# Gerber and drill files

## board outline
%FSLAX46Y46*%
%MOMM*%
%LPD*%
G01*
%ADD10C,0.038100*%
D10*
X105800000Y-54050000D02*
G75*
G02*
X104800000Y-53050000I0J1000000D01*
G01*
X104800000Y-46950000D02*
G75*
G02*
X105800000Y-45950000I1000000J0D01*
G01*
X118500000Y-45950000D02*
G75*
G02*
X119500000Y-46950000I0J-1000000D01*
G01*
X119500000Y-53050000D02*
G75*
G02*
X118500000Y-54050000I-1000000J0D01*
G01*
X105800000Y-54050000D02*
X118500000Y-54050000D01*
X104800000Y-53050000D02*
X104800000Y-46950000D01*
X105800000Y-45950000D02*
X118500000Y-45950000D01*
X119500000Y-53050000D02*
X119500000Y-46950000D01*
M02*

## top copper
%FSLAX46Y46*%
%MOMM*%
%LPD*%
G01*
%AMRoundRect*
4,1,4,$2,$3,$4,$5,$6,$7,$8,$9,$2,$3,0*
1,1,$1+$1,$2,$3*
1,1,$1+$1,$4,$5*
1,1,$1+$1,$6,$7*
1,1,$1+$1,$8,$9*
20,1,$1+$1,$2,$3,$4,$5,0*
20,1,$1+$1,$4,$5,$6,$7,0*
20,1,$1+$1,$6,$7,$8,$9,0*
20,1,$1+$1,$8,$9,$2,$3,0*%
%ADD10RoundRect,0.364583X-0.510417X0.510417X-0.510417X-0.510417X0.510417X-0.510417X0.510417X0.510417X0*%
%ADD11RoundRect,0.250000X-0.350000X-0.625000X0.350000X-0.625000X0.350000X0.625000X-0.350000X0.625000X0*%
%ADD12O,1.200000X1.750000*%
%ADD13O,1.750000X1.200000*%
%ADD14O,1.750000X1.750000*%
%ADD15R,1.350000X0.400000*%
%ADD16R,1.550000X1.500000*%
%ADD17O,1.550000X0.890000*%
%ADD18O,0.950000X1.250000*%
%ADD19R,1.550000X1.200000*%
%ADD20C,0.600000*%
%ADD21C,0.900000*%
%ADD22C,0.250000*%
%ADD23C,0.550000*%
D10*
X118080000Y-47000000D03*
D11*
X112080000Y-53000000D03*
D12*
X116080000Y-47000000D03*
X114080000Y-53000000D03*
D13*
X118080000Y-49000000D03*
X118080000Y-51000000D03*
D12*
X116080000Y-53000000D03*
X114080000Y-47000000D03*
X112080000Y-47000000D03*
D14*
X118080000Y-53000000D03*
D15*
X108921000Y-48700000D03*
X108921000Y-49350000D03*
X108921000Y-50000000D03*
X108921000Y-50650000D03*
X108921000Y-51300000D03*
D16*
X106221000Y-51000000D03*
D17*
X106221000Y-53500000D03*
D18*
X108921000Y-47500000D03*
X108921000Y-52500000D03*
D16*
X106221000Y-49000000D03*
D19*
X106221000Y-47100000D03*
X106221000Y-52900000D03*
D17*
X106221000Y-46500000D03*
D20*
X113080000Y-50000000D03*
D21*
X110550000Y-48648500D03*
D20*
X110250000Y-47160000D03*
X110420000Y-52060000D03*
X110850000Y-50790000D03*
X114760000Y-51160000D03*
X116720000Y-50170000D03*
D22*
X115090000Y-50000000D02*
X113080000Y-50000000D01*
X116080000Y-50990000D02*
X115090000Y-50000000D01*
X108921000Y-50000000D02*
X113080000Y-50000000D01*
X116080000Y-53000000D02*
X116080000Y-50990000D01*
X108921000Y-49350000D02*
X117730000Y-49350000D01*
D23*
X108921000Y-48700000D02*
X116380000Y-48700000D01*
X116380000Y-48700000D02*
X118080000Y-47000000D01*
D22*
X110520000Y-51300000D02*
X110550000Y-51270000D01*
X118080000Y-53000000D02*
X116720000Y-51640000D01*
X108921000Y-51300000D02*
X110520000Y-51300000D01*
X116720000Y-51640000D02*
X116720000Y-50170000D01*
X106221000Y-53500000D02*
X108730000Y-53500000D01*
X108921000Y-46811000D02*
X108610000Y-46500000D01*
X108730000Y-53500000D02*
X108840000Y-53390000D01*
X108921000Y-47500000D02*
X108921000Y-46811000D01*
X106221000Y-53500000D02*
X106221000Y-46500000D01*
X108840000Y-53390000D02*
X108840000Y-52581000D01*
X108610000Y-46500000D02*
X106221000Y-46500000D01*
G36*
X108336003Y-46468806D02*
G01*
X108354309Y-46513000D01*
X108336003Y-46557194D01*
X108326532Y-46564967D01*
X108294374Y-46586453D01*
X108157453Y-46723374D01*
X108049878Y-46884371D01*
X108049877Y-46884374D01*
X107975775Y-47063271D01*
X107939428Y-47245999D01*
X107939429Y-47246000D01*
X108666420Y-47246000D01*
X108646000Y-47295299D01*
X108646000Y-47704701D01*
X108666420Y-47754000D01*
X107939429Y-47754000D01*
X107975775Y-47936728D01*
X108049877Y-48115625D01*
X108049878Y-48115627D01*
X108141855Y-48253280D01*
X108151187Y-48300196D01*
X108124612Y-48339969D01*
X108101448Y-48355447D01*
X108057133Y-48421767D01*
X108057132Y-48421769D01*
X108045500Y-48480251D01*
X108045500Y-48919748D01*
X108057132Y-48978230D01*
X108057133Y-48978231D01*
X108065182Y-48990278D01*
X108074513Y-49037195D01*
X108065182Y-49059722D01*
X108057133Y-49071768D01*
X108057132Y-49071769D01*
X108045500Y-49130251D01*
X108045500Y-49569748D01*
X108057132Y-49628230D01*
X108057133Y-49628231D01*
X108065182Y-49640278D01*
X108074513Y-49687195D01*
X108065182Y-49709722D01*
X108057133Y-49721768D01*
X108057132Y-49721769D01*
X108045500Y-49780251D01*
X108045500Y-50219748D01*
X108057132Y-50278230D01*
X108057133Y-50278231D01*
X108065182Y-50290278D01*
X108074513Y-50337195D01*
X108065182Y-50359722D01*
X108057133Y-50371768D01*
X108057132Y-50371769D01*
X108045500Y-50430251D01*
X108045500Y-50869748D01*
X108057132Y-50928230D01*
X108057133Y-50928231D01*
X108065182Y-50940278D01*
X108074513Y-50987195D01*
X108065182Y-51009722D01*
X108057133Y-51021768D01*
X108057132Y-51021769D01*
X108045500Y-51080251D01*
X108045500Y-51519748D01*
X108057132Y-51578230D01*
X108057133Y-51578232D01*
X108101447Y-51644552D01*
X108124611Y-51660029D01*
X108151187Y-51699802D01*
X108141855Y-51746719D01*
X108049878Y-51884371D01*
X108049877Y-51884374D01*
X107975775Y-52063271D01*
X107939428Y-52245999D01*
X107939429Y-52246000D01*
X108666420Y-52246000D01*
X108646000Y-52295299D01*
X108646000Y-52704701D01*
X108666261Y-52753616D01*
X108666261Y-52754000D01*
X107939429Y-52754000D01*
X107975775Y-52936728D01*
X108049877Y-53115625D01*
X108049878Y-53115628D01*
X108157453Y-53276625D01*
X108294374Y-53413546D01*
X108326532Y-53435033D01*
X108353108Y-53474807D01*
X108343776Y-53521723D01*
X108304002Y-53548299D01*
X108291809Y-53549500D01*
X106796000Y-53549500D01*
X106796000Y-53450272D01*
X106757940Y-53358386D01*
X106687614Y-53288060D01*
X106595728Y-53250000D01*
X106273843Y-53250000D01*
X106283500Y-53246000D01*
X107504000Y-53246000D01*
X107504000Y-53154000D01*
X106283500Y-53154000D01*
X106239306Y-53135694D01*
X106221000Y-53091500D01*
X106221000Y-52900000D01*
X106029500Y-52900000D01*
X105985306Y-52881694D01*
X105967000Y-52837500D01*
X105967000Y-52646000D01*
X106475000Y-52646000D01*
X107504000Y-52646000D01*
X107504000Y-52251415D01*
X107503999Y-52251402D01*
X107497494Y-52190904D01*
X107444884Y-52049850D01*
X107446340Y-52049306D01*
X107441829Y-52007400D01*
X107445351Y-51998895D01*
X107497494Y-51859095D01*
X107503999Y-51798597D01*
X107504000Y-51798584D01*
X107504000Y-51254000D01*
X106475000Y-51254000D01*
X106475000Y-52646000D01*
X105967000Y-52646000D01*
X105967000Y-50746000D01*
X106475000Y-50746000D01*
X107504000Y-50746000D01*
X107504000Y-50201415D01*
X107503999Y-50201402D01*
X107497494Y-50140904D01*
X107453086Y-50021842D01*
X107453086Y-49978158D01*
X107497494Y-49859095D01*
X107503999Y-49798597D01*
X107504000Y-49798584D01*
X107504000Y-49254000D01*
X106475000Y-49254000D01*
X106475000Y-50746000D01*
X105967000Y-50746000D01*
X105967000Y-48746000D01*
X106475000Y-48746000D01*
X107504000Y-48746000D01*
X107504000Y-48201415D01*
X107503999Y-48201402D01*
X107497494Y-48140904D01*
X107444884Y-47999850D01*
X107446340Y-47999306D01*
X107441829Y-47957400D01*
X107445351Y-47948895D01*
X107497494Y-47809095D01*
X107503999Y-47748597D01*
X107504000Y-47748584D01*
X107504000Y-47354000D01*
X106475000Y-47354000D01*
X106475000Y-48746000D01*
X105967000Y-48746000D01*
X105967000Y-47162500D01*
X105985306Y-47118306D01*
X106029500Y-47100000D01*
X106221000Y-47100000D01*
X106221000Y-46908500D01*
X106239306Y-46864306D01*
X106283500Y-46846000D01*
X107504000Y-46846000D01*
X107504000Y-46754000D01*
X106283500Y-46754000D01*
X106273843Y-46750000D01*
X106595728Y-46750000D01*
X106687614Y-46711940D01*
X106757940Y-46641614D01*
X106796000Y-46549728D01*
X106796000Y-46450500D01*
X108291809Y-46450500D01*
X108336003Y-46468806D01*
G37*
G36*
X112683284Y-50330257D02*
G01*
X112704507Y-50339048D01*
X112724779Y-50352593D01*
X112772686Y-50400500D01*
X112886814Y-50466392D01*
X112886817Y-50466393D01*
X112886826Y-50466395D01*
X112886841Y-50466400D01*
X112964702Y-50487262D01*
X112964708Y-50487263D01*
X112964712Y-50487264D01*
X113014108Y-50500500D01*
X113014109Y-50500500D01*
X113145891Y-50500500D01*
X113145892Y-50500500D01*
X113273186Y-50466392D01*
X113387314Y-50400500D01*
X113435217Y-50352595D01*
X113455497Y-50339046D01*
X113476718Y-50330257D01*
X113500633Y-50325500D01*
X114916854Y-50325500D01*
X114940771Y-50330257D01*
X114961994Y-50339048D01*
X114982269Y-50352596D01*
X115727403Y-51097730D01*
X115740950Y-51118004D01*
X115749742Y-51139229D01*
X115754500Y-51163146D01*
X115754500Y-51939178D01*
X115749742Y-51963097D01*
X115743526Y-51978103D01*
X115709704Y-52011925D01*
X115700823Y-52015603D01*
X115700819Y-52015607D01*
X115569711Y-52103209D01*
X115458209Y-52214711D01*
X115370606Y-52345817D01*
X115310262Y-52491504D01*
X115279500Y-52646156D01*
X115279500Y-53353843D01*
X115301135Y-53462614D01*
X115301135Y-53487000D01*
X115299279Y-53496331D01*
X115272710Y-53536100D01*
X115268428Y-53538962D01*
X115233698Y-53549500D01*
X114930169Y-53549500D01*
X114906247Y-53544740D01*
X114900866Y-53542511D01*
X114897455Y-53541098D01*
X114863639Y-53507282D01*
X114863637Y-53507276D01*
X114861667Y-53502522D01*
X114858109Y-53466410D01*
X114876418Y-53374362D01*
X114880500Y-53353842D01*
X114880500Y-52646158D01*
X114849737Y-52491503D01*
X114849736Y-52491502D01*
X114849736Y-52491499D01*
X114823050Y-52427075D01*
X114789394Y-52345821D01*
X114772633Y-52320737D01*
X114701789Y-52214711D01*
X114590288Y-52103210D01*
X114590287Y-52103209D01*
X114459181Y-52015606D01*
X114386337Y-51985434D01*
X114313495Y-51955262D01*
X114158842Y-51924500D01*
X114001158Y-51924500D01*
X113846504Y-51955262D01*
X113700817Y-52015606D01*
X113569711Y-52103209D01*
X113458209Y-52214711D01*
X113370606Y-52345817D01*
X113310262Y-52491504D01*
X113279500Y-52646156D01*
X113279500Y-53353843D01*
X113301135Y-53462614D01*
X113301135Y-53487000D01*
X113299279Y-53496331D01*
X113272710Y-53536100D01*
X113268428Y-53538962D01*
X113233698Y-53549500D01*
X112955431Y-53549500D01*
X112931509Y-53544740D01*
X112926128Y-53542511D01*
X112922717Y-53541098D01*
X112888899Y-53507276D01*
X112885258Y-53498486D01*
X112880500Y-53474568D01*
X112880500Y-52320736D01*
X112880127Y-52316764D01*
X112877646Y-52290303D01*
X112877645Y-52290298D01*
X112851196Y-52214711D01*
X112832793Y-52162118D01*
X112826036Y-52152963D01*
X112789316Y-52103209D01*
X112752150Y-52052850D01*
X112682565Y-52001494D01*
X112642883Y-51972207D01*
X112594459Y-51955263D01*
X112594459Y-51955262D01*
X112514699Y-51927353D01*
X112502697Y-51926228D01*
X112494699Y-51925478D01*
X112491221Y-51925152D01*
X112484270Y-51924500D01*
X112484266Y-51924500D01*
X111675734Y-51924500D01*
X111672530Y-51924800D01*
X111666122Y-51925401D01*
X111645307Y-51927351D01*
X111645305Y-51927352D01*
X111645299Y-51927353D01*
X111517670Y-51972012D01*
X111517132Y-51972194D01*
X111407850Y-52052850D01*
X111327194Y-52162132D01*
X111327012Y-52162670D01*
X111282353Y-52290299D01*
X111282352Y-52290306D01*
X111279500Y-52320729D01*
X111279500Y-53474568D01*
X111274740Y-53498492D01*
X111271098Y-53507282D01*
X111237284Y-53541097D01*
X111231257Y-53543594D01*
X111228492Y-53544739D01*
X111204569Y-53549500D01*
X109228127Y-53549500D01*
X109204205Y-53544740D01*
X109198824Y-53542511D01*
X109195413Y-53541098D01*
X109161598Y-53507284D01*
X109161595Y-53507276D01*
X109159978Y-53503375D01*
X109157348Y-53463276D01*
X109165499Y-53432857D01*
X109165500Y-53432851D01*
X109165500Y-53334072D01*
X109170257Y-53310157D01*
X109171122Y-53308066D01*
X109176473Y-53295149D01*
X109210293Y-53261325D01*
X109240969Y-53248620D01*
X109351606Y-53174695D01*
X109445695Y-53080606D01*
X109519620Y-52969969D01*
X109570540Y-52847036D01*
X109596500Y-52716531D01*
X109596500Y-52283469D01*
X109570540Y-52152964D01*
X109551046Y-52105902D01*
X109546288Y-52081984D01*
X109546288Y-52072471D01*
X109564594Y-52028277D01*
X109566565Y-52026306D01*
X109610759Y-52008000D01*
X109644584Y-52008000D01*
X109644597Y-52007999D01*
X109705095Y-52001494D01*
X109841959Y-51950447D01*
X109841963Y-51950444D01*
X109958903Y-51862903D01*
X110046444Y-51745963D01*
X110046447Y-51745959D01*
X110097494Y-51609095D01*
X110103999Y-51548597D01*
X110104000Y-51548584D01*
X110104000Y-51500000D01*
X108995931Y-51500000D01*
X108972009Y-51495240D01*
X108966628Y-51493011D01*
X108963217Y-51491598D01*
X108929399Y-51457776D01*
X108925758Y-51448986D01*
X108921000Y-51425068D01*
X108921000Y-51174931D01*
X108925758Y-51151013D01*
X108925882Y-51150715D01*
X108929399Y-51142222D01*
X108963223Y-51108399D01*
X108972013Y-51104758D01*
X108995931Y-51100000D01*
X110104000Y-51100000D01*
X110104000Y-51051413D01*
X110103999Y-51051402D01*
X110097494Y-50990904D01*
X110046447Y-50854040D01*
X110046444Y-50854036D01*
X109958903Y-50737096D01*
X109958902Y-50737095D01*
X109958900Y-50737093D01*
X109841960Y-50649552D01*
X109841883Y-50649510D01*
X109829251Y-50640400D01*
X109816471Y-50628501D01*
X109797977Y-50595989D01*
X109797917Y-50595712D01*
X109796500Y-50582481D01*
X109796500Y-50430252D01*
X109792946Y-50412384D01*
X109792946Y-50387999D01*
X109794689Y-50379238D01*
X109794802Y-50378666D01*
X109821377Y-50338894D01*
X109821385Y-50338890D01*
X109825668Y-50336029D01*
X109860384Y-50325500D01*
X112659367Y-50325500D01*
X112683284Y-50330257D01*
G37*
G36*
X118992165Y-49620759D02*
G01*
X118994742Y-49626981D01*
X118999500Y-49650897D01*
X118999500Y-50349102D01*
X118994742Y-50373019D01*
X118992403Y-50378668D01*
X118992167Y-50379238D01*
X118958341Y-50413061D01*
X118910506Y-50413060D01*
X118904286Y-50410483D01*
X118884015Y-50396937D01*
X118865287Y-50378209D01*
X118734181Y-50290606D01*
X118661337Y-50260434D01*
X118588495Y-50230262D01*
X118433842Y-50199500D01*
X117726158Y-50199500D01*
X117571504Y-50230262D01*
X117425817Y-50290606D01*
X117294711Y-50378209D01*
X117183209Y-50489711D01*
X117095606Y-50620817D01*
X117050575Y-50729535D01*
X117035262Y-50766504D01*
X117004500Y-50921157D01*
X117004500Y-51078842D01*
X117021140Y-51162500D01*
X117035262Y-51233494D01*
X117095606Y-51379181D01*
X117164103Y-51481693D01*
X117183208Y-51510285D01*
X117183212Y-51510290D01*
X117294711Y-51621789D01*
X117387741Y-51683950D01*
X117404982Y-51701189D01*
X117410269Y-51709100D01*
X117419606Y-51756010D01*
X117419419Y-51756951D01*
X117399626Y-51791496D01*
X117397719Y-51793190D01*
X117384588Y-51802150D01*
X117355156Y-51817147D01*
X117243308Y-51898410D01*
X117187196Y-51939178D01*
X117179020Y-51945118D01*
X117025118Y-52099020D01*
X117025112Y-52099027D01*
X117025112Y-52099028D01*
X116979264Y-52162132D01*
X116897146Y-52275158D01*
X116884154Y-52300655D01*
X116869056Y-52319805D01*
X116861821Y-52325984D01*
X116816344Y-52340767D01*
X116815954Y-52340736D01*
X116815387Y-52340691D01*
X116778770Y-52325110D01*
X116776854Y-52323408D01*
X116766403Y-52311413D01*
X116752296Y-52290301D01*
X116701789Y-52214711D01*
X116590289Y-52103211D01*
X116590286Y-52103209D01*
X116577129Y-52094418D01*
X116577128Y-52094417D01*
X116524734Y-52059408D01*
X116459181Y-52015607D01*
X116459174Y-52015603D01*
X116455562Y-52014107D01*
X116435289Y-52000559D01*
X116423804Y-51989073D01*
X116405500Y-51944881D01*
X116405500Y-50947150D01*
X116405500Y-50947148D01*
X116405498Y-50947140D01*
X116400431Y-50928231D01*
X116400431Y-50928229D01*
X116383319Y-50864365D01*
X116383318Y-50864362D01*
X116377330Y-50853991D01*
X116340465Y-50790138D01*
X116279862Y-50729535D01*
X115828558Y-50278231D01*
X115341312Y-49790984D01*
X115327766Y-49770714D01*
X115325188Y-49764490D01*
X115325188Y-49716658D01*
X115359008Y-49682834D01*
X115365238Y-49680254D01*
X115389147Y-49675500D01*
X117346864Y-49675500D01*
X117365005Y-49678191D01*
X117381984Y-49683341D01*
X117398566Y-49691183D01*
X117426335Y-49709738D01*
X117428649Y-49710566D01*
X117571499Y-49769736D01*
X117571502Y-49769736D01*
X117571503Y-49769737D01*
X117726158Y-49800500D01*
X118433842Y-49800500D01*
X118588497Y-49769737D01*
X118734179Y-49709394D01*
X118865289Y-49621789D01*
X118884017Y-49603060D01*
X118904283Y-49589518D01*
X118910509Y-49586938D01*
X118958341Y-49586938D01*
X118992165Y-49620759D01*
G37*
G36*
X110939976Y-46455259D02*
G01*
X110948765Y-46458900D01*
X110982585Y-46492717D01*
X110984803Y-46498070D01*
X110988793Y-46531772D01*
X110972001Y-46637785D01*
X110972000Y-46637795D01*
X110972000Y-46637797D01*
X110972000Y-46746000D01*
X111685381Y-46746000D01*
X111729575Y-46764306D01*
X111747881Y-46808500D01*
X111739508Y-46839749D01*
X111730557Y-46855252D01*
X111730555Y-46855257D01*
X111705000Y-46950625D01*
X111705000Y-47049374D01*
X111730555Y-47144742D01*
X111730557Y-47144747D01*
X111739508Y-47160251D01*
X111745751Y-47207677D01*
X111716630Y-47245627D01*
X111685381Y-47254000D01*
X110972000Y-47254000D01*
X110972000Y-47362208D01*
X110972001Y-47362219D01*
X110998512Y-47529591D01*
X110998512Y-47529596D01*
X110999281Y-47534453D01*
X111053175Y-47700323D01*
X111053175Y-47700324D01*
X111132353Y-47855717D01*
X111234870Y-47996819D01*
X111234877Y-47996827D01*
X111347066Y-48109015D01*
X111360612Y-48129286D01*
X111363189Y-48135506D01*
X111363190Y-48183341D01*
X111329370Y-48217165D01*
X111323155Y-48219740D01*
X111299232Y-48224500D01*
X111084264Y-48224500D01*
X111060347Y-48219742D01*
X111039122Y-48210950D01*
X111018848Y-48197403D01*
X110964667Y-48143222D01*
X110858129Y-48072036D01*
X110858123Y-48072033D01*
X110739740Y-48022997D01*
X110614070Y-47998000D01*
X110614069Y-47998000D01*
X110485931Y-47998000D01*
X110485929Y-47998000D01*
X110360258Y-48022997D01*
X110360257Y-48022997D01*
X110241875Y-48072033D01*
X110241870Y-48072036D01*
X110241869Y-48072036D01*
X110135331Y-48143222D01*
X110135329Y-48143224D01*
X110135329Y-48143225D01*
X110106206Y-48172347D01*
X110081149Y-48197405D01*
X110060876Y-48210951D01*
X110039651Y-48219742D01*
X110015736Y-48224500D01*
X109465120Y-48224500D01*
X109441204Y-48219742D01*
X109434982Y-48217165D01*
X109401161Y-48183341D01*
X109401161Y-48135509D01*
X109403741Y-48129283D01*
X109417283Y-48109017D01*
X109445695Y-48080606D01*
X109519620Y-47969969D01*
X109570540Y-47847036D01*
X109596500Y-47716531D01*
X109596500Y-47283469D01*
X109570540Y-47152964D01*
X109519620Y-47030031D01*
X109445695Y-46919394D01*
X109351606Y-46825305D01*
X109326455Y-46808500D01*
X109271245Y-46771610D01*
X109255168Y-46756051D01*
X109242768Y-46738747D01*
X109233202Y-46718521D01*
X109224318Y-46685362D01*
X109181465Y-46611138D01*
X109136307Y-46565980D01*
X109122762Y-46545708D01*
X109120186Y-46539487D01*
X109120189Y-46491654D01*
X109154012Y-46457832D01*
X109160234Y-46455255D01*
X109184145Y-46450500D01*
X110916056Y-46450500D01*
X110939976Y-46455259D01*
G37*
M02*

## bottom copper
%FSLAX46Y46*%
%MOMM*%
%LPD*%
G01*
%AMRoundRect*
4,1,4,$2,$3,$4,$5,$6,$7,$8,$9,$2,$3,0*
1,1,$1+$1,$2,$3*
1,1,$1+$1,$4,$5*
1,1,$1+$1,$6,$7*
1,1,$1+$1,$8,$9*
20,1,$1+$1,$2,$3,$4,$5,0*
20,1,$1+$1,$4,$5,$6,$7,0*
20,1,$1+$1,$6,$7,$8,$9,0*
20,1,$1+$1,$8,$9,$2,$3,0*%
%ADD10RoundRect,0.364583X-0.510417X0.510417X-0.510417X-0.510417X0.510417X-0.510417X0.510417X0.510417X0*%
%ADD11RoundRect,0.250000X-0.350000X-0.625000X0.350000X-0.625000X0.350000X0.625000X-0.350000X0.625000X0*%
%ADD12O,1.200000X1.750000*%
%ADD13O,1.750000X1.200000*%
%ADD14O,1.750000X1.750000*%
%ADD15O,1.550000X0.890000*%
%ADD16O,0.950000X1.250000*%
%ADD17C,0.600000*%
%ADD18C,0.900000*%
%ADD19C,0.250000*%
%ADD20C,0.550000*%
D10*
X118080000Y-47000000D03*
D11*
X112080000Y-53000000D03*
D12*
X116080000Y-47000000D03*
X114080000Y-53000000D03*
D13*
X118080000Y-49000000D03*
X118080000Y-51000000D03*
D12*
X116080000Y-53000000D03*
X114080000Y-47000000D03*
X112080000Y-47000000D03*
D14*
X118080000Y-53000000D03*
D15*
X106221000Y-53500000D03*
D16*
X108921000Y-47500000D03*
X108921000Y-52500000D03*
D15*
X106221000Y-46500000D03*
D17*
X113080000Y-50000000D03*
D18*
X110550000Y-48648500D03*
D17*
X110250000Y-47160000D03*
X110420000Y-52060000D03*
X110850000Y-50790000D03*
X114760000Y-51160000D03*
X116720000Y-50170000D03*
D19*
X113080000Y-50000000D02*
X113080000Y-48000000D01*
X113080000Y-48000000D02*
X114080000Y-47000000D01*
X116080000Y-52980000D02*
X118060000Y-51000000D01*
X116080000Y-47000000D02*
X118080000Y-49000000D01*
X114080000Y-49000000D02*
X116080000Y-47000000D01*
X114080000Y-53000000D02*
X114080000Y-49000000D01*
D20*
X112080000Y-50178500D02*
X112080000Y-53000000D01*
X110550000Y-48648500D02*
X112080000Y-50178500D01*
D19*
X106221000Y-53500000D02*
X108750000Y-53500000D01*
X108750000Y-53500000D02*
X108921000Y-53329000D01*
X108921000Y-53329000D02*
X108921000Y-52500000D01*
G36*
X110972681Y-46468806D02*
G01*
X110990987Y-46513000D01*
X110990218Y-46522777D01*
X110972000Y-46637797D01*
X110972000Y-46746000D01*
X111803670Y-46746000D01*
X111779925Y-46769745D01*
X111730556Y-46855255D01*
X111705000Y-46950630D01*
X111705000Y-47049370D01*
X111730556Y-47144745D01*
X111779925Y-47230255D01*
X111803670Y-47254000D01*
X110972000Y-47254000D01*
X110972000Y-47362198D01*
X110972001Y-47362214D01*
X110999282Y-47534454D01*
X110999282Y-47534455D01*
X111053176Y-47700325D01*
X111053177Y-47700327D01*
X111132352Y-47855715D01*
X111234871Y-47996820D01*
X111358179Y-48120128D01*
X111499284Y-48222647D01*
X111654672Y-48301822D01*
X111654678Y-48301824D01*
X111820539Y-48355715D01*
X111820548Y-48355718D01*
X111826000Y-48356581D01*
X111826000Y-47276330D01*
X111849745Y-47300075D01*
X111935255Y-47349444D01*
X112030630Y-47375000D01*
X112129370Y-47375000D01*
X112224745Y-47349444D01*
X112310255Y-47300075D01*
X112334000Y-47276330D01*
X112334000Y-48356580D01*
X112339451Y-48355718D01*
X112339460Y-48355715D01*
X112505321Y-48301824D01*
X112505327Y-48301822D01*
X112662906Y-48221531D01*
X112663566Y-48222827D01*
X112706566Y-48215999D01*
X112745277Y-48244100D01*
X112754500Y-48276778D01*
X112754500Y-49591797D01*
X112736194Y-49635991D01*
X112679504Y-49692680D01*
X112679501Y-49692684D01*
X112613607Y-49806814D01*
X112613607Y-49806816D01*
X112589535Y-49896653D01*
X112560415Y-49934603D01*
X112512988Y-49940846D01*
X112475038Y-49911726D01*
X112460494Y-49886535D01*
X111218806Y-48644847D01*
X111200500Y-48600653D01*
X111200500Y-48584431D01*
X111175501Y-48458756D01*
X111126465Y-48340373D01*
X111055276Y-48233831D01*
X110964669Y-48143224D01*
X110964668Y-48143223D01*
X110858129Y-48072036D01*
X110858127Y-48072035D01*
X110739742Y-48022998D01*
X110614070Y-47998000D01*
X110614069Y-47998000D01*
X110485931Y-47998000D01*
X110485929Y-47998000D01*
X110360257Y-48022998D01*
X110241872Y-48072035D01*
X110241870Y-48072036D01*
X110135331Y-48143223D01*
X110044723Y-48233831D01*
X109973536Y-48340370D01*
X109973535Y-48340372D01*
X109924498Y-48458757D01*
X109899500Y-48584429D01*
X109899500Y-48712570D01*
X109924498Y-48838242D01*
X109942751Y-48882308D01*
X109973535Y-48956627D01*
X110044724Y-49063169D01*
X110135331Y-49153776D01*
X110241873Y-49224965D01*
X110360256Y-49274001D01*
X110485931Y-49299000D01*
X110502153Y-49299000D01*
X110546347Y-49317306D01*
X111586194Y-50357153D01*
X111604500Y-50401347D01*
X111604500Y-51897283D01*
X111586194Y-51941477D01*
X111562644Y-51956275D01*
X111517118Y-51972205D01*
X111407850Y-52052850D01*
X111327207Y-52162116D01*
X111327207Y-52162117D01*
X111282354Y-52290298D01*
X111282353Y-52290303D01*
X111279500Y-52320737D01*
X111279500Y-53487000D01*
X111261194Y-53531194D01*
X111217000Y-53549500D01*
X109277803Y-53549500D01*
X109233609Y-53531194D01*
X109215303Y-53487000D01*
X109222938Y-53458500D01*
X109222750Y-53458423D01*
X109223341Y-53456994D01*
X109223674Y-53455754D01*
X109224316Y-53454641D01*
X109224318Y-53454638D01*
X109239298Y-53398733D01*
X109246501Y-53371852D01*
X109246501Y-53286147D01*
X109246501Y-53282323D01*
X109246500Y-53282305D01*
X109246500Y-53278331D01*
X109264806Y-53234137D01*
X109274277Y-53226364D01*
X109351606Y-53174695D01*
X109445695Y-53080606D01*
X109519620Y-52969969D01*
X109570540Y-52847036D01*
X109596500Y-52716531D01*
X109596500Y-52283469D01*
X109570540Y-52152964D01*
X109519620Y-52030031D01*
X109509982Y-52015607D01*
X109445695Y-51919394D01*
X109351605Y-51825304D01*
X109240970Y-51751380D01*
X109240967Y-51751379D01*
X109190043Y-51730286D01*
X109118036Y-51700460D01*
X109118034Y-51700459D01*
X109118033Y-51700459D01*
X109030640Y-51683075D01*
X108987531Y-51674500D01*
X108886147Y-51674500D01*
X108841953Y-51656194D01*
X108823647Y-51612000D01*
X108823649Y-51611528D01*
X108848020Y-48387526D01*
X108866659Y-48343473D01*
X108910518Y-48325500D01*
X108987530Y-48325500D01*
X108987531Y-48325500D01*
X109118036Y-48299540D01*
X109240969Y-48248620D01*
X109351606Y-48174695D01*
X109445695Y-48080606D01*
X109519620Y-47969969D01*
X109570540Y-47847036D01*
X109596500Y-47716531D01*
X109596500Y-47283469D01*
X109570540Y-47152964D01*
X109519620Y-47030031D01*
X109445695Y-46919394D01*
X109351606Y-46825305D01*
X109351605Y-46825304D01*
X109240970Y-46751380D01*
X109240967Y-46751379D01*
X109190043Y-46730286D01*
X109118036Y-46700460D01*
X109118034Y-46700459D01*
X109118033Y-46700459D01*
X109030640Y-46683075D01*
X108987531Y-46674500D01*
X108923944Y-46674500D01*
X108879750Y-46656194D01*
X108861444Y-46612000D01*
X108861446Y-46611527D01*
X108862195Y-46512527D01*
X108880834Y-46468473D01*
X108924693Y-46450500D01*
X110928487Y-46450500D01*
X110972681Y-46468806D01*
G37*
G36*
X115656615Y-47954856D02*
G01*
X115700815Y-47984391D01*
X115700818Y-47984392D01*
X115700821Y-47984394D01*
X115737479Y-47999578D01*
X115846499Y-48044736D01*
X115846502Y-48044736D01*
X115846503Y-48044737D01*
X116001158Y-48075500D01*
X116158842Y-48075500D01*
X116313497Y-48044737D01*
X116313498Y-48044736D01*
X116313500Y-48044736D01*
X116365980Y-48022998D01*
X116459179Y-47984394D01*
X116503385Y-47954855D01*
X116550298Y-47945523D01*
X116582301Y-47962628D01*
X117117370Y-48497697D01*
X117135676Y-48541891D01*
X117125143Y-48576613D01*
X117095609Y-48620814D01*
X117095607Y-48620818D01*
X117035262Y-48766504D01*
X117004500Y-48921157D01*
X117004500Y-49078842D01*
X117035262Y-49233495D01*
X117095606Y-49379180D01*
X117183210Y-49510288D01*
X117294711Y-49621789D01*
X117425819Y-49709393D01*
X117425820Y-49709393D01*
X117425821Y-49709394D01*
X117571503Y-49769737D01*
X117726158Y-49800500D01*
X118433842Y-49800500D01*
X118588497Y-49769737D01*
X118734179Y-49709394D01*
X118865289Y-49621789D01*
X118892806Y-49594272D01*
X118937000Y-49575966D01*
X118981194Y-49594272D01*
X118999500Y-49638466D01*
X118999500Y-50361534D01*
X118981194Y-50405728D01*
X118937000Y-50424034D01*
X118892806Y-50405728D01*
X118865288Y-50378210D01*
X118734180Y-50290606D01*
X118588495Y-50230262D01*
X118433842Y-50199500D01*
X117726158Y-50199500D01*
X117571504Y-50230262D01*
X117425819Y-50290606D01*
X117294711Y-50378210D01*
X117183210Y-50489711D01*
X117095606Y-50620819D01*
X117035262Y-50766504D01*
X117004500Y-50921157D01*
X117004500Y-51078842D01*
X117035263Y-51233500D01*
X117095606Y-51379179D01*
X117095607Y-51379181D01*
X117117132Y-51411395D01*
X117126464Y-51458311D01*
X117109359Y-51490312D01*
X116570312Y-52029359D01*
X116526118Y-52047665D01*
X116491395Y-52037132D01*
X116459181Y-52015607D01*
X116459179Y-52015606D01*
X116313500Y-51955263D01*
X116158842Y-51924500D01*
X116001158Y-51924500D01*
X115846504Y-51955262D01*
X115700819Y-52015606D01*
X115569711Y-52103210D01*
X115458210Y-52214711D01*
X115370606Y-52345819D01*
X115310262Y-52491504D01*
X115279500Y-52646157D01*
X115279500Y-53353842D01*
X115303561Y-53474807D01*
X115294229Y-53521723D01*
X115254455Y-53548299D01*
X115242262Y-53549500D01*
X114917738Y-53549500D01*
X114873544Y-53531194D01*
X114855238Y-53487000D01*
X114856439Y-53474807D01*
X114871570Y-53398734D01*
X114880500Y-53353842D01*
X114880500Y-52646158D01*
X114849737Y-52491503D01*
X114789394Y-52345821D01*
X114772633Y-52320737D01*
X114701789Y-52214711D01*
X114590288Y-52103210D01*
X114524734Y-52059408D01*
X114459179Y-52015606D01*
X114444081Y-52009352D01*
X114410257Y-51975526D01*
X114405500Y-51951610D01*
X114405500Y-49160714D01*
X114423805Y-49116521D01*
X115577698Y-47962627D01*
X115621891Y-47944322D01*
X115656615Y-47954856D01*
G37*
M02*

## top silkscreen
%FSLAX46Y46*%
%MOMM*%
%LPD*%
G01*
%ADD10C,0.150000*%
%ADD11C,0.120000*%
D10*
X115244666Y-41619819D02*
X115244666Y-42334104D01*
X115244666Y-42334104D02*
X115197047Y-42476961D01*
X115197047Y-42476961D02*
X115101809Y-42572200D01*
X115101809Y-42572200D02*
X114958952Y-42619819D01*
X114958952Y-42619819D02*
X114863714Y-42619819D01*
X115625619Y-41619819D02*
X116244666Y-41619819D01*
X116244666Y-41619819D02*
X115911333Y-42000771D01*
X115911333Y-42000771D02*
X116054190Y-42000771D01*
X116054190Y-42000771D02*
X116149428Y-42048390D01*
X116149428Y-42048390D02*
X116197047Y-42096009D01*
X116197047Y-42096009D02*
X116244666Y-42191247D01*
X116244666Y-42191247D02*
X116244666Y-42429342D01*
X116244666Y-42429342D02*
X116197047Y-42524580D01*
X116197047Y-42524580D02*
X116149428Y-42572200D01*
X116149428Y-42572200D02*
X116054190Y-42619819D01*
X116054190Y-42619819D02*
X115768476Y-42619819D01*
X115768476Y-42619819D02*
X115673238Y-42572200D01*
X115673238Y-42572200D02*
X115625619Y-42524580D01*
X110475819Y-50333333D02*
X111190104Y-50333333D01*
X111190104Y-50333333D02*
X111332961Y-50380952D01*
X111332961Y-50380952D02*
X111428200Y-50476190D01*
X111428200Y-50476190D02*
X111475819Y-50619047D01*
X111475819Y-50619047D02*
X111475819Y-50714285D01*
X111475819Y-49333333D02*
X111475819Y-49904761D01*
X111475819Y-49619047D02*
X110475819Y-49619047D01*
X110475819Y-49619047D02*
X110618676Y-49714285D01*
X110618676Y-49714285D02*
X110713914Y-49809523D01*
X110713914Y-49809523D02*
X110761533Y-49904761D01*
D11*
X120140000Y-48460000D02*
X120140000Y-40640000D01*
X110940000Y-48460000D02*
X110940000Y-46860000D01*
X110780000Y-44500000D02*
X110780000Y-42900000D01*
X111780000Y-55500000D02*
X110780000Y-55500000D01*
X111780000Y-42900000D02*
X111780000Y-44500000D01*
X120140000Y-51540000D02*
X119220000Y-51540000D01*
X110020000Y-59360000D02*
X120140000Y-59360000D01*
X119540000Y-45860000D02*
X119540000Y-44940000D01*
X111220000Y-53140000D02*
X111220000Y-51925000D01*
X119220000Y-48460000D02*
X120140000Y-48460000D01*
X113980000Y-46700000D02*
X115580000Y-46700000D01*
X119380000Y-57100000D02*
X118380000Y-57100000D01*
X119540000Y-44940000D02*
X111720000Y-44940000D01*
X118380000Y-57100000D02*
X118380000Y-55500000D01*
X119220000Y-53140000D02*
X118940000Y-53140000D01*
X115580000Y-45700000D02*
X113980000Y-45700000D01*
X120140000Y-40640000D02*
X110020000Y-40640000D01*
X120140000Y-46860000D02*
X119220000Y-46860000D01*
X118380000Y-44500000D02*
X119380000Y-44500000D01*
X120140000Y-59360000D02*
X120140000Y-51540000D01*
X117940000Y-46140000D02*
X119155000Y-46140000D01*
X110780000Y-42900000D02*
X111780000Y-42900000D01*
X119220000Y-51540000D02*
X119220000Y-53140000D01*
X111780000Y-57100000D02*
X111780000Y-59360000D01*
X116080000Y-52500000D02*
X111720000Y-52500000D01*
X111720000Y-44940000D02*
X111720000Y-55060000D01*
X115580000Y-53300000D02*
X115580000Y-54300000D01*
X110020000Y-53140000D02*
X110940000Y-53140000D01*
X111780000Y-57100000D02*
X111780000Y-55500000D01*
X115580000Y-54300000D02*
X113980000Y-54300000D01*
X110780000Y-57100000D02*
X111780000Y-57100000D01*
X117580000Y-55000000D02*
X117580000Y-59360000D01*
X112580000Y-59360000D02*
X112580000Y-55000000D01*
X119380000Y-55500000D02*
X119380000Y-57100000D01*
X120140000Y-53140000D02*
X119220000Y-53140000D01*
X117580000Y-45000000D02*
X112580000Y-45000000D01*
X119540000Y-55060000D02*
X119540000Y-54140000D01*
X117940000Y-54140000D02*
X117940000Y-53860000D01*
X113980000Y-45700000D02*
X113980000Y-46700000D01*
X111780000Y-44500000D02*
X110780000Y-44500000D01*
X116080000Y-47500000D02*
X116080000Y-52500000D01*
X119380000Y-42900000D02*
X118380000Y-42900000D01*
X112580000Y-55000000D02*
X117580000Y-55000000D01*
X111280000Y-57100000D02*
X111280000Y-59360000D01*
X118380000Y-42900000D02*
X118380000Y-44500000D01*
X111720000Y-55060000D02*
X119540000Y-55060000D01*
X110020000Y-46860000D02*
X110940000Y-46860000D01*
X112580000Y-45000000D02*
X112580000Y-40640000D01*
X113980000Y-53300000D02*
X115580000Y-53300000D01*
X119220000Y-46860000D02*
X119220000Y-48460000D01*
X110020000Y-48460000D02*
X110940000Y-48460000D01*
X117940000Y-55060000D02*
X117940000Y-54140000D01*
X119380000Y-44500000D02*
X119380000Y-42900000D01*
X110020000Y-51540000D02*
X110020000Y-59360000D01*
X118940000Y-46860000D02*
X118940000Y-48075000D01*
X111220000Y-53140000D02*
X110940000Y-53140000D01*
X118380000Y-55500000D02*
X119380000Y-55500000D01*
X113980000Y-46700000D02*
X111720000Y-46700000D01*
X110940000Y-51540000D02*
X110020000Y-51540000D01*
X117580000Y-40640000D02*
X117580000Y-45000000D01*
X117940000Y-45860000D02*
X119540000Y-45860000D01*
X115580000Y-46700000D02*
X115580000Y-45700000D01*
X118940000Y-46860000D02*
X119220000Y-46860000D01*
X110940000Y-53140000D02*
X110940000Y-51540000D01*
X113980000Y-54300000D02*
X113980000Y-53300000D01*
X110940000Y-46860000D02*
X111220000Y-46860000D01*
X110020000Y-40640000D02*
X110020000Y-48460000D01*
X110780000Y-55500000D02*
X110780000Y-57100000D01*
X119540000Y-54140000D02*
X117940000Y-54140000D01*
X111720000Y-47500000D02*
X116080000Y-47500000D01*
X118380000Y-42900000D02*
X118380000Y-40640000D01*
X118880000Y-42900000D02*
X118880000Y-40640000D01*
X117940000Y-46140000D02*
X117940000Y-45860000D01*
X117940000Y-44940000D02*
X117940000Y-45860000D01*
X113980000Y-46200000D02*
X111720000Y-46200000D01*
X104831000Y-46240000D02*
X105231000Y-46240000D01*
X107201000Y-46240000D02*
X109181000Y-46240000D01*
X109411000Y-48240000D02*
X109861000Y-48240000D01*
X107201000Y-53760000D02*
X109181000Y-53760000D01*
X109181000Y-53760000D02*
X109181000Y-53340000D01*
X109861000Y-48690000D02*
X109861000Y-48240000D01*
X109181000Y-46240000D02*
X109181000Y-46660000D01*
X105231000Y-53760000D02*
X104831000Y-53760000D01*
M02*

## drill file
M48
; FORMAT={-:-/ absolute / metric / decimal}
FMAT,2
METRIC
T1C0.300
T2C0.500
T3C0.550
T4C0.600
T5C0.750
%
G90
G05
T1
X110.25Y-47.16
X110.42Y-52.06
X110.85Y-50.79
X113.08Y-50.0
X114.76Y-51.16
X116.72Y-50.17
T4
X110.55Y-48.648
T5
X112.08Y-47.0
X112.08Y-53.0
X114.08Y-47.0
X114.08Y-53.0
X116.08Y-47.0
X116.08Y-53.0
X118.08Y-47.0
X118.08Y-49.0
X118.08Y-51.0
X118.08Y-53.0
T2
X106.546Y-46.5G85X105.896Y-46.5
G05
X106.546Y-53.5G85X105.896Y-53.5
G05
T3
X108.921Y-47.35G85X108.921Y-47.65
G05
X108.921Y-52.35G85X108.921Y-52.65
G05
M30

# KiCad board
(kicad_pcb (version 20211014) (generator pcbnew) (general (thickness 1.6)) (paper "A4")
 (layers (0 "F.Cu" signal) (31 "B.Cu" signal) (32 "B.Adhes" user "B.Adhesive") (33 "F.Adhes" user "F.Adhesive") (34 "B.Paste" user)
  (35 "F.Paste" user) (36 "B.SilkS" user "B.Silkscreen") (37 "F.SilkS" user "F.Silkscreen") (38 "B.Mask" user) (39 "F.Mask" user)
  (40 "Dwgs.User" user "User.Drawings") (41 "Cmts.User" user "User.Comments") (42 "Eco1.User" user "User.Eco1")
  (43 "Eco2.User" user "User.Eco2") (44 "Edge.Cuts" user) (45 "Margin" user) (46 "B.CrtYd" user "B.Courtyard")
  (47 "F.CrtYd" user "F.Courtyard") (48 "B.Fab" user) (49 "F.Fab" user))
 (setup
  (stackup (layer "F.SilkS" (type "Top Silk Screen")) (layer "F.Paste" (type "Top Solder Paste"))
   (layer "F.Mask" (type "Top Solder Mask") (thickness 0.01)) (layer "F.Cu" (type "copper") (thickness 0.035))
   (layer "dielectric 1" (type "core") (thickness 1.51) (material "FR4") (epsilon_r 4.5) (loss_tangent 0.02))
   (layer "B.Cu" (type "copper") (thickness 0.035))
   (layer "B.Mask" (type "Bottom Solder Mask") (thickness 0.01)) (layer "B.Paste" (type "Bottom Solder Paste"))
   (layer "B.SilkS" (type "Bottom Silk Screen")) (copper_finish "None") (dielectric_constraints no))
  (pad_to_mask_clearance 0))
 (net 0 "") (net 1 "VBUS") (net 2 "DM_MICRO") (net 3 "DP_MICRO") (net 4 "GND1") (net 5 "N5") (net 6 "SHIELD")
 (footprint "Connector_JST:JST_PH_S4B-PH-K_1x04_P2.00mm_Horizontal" (layer "F.Cu") (at 118.08 47 180)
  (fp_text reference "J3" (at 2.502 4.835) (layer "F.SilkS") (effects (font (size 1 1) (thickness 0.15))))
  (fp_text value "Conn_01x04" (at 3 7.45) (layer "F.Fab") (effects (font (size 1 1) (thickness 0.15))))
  (fp_line (start -2.06 -1.46) (end -2.06 6.36) (layer "F.SilkS") (width 0.12))
  (fp_line (start 7.14 -1.46) (end 7.14 0.14) (layer "F.SilkS") (width 0.12))
  (fp_line (start 7.3 2.5) (end 7.3 4.1) (layer "F.SilkS") (width 0.12))
  (fp_line (start 6.3 -8.5) (end 7.3 -8.5) (layer "F.SilkS") (width 0.12))
  (fp_line (start 6.3 4.1) (end 6.3 2.5) (layer "F.SilkS") (width 0.12))
  (fp_line (start -2.06 -4.54) (end -1.14 -4.54) (layer "F.SilkS") (width 0.12))
  (fp_line (start 8.06 -12.36) (end -2.06 -12.36) (layer "F.SilkS") (width 0.12))
  (fp_line (start -1.46 1.14) (end -1.46 2.06) (layer "F.SilkS") (width 0.12))
  (fp_line (start 6.86 -6.14) (end 6.86 -4.925) (layer "F.SilkS") (width 0.12))
  (fp_line (start -1.14 -1.46) (end -2.06 -1.46) (layer "F.SilkS") (width 0.12))
  (fp_line (start 4.1 0.3) (end 2.5 0.3) (layer "F.SilkS") (width 0.12))
  (fp_line (start -1.3 -10.1) (end -0.3 -10.1) (layer "F.SilkS") (width 0.12))
  (fp_line (start -1.46 2.06) (end 6.36 2.06) (layer "F.SilkS") (width 0.12))
  (fp_line (start -0.3 -10.1) (end -0.3 -8.5) (layer "F.SilkS") (width 0.12))
  (fp_line (start -1.14 -6.14) (end -0.86 -6.14) (layer "F.SilkS") (width 0.12))
  (fp_line (start 2.5 1.3) (end 4.1 1.3) (layer "F.SilkS") (width 0.12))
  (fp_line (start -2.06 6.36) (end 8.06 6.36) (layer "F.SilkS") (width 0.12))
  (fp_line (start -2.06 0.14) (end -1.14 0.14) (layer "F.SilkS") (width 0.12))
  (fp_line (start -0.3 2.5) (end -1.3 2.5) (layer "F.SilkS") (width 0.12))
  (fp_line (start -2.06 -12.36) (end -2.06 -4.54) (layer "F.SilkS") (width 0.12))
  (fp_line (start 0.14 0.86) (end -1.075 0.86) (layer "F.SilkS") (width 0.12))
  (fp_line (start 7.3 4.1) (end 6.3 4.1) (layer "F.SilkS") (width 0.12))
  (fp_line (start -1.14 -4.54) (end -1.14 -6.14) (layer "F.SilkS") (width 0.12))
  (fp_line (start 6.3 -10.1) (end 6.3 -12.36) (layer "F.SilkS") (width 0.12))
  (fp_line (start 2 -5.5) (end 6.36 -5.5) (layer "F.SilkS") (width 0.12))
  (fp_line (start 6.36 2.06) (end 6.36 -8.06) (layer "F.SilkS") (width 0.12))
  (fp_line (start 2.5 -6.3) (end 2.5 -7.3) (layer "F.SilkS") (width 0.12))
  (fp_line (start 8.06 -6.14) (end 7.14 -6.14) (layer "F.SilkS") (width 0.12))
  (fp_line (start 6.3 -10.1) (end 6.3 -8.5) (layer "F.SilkS") (width 0.12))
  (fp_line (start 2.5 -7.3) (end 4.1 -7.3) (layer "F.SilkS") (width 0.12))
  (fp_line (start 7.3 -10.1) (end 6.3 -10.1) (layer "F.SilkS") (width 0.12))
  (fp_line (start 0.5 -8) (end 0.5 -12.36) (layer "F.SilkS") (width 0.12))
  (fp_line (start 5.5 -12.36) (end 5.5 -8) (layer "F.SilkS") (width 0.12))
  (fp_line (start -1.3 -8.5) (end -1.3 -10.1) (layer "F.SilkS") (width 0.12))
  (fp_line (start -2.06 -6.14) (end -1.14 -6.14) (layer "F.SilkS") (width 0.12))
  (fp_line (start 0.5 2) (end 5.5 2) (layer "F.SilkS") (width 0.12))
  (fp_line (start -1.46 -8.06) (end -1.46 -7.14) (layer "F.SilkS") (width 0.12))
  (fp_line (start 0.14 -7.14) (end 0.14 -6.86) (layer "F.SilkS") (width 0.12))
  (fp_line (start 4.1 1.3) (end 4.1 0.3) (layer "F.SilkS") (width 0.12))
  (fp_line (start 6.3 2.5) (end 7.3 2.5) (layer "F.SilkS") (width 0.12))
  (fp_line (start 2 -0.5) (end 2 -5.5) (layer "F.SilkS") (width 0.12))
  (fp_line (start -1.3 4.1) (end -0.3 4.1) (layer "F.SilkS") (width 0.12))
  (fp_line (start 5.5 -8) (end 0.5 -8) (layer "F.SilkS") (width 0.12))
  (fp_line (start 6.8 -10.1) (end 6.8 -12.36) (layer "F.SilkS") (width 0.12))
  (fp_line (start -0.3 4.1) (end -0.3 2.5) (layer "F.SilkS") (width 0.12))
  (fp_line (start 6.36 -8.06) (end -1.46 -8.06) (layer "F.SilkS") (width 0.12))
  (fp_line (start 8.06 0.14) (end 7.14 0.14) (layer "F.SilkS") (width 0.12))
  (fp_line (start 5.5 2) (end 5.5 6.36) (layer "F.SilkS") (width 0.12))
  (fp_line (start 4.1 -6.3) (end 2.5 -6.3) (layer "F.SilkS") (width 0.12))
  (fp_line (start -1.14 0.14) (end -1.14 -1.46) (layer "F.SilkS") (width 0.12))
  (fp_line (start 8.06 -1.46) (end 7.14 -1.46) (layer "F.SilkS") (width 0.12))
  (fp_line (start 0.14 -8.06) (end 0.14 -7.14) (layer "F.SilkS") (width 0.12))
  (fp_line (start -1.3 2.5) (end -1.3 4.1) (layer "F.SilkS") (width 0.12))
  (fp_line (start 8.06 -4.54) (end 8.06 -12.36) (layer "F.SilkS") (width 0.12))
  (fp_line (start -0.86 0.14) (end -0.86 -1.075) (layer "F.SilkS") (width 0.12))
  (fp_line (start 6.86 -6.14) (end 7.14 -6.14) (layer "F.SilkS") (width 0.12))
  (fp_line (start -0.3 -8.5) (end -1.3 -8.5) (layer "F.SilkS") (width 0.12))
  (fp_line (start 4.1 0.3) (end 6.36 0.3) (layer "F.SilkS") (width 0.12))
  (fp_line (start 7.14 -4.54) (end 8.06 -4.54) (layer "F.SilkS") (width 0.12))
  (fp_line (start 0.5 6.36) (end 0.5 2) (layer "F.SilkS") (width 0.12))
  (fp_line (start 0.14 1.14) (end -1.46 1.14) (layer "F.SilkS") (width 0.12))
  (fp_line (start 2.5 0.3) (end 2.5 1.3) (layer "F.SilkS") (width 0.12))
  (fp_line (start -0.86 0.14) (end -1.14 0.14) (layer "F.SilkS") (width 0.12))
  (fp_line (start 7.14 -6.14) (end 7.14 -4.54) (layer "F.SilkS") (width 0.12))
  (fp_line (start 4.1 -7.3) (end 4.1 -6.3) (layer "F.SilkS") (width 0.12))
  (fp_line (start 7.14 0.14) (end 6.86 0.14) (layer "F.SilkS") (width 0.12))
  (fp_line (start 8.06 6.36) (end 8.06 -1.46) (layer "F.SilkS") (width 0.12))
  (fp_line (start 7.3 -8.5) (end 7.3 -10.1) (layer "F.SilkS") (width 0.12))
  (fp_line (start -1.46 -7.14) (end 0.14 -7.14) (layer "F.SilkS") (width 0.12))
  (fp_line (start 6.36 -0.5) (end 2 -0.5) (layer "F.SilkS") (width 0.12))
  (fp_line (start -0.3 4.1) (end -0.3 6.36) (layer "F.SilkS") (width 0.12))
  (fp_line (start -0.8 4.1) (end -0.8 6.36) (layer "F.SilkS") (width 0.12))
  (fp_line (start 0.14 0.86) (end 0.14 1.14) (layer "F.SilkS") (width 0.12))
  (fp_line (start 0.14 2.06) (end 0.14 1.14) (layer "F.SilkS") (width 0.12))
  (fp_line (start 4.1 0.8) (end 6.36 0.8) (layer "F.SilkS") (width 0.12))
  (pad "1" thru_hole roundrect (at 0 0 270) (size 1.75 1.75) (drill 0.75) (layers *.Cu *.Mask) (roundrect_rratio 0.2083331429)
   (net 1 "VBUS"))
  (pad "1" thru_hole roundrect (at 6 -6) (size 1.2 1.75) (drill 0.75) (layers *.Cu *.Mask) (roundrect_rratio 0.2083333333) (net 1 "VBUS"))
  (pad "2" thru_hole oval (at 2 0 180) (size 1.2 1.75) (drill 0.75) (layers *.Cu *.Mask) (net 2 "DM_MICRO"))
  (pad "2" thru_hole oval (at 4 -6) (size 1.2 1.75) (drill 0.75) (layers *.Cu *.Mask) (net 2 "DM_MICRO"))
  (pad "2" thru_hole oval (at 0 -2 270) (size 1.2 1.75) (drill 0.75) (layers *.Cu *.Mask) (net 2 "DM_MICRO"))
  (pad "3" thru_hole oval (at 0 -4 270) (size 1.2 1.75) (drill 0.75) (layers *.Cu *.Mask) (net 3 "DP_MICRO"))
  (pad "3" thru_hole oval (at 2 -6) (size 1.2 1.75) (drill 0.75) (layers *.Cu *.Mask) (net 3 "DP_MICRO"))
  (pad "3" thru_hole oval (at 4 0 180) (size 1.2 1.75) (drill 0.75) (layers *.Cu *.Mask) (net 3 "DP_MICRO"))
  (pad "4" thru_hole oval (at 6 0 180) (size 1.2 1.75) (drill 0.75) (layers *.Cu *.Mask) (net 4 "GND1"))
  (pad "4" thru_hole oval (at 0 -6 270) (size 1.75 1.75) (drill 0.75) (layers *.Cu *.Mask) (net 4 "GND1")))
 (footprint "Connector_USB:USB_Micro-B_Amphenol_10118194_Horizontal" (layer "F.Cu") (at 107.521 50 -90)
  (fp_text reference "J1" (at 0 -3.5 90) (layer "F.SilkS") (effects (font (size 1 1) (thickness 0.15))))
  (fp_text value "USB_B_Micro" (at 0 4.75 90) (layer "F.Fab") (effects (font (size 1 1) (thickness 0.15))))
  (fp_line (start -3.76 2.69) (end -3.76 2.29) (layer "F.SilkS") (width 0.12))
  (fp_line (start -3.76 0.32) (end -3.76 -1.66) (layer "F.SilkS") (width 0.12))
  (fp_line (start -1.76 -1.89) (end -1.76 -2.34) (layer "F.SilkS") (width 0.12))
  (fp_line (start 3.76 0.32) (end 3.76 -1.66) (layer "F.SilkS") (width 0.12))
  (fp_line (start 3.76 -1.66) (end 3.34 -1.66) (layer "F.SilkS") (width 0.12))
  (fp_line (start -1.31 -2.34) (end -1.76 -2.34) (layer "F.SilkS") (width 0.12))
  (fp_line (start -3.76 -1.66) (end -3.34 -1.66) (layer "F.SilkS") (width 0.12))
  (fp_line (start 3.76 2.29) (end 3.76 2.69) (layer "F.SilkS") (width 0.12))
  (pad "" smd oval (at 2.5 -1.4 270) (size 1.25 0.95) (layers "F.Paste"))
  (pad "" smd oval (at -3.5 1.3 270) (size 0.89 1.55) (layers "F.Paste"))
  (pad "" smd oval (at 3.5 1.3 270) (size 0.89 1.55) (layers "F.Paste"))
  (pad "" smd oval (at -2.5 -1.4 270) (size 1.25 0.95) (layers "F.Paste"))
  (pad "1" smd rect (at -1.3 -1.4 270) (size 0.4 1.35) (layers "F.Cu" "F.Paste" "F.Mask") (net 1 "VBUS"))
  (pad "2" smd rect (at -0.65 -1.4 270) (size 0.4 1.35) (layers "F.Cu" "F.Paste" "F.Mask") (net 2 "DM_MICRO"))
  (pad "3" smd rect (at 0 -1.4 270) (size 0.4 1.35) (layers "F.Cu" "F.Paste" "F.Mask") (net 3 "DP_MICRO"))
  (pad "4" smd rect (at 0.65 -1.4 270) (size 0.4 1.35) (layers "F.Cu" "F.Paste" "F.Mask") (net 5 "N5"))
  (pad "5" smd rect (at 1.3 -1.4 270) (size 0.4 1.35) (layers "F.Cu" "F.Paste" "F.Mask") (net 4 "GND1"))
  (pad "6" smd rect (at 1 1.3 270) (size 1.5 1.55) (layers "F.Cu" "F.Paste" "F.Mask") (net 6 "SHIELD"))
  (pad "6" thru_hole oval (at 3.5 1.3 270) (size 0.89 1.55) (drill oval 0.5 1.15) (layers *.Cu *.Mask) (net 6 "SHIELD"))
  (pad "6" thru_hole oval (at -2.5 -1.4 270) (size 1.25 0.95) (drill oval 0.85 0.55) (layers *.Cu *.Mask) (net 6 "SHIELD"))
  (pad "6" thru_hole oval (at 2.5 -1.4 270) (size 1.25 0.95) (drill oval 0.85 0.55) (layers *.Cu *.Mask) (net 6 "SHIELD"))
  (pad "6" smd rect (at -1 1.3 270) (size 1.5 1.55) (layers "F.Cu" "F.Paste" "F.Mask") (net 6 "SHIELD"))
  (pad "6" smd rect (at -2.9 1.3 270) (size 1.2 1.55) (layers "F.Cu" "F.Paste" "F.Mask") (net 6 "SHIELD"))
  (pad "6" smd rect (at 2.9 1.3 270) (size 1.2 1.55) (layers "F.Cu" "F.Paste" "F.Mask") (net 6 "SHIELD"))
  (pad "6" thru_hole oval (at -3.5 1.3 270) (size 0.89 1.55) (drill oval 0.5 1.15) (layers *.Cu *.Mask) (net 6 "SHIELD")))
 (gr_arc (start 105.8 54.05) (mid 105.092893 53.757107) (end 104.8 53.05) (layer "Edge.Cuts") (width 0.0381))
 (gr_arc (start 104.8 46.95) (mid 105.092893 46.242893) (end 105.8 45.95) (layer "Edge.Cuts") (width 0.0381))
 (gr_arc (start 118.5 45.95) (mid 119.207107 46.242893) (end 119.5 46.95) (layer "Edge.Cuts") (width 0.0381))
 (gr_arc (start 119.5 53.05) (mid 119.207107 53.757107) (end 118.5 54.05) (layer "Edge.Cuts") (width 0.0381))
 (gr_line (start 105.8 54.05) (end 118.5 54.05) (layer "Edge.Cuts") (width 0.0381))
 (gr_line (start 104.8 53.05) (end 104.8 46.95) (layer "Edge.Cuts") (width 0.0381))
 (gr_line (start 105.8 45.95) (end 118.5 45.95) (layer "Edge.Cuts") (width 0.0381))
 (gr_line (start 119.5 53.05) (end 119.5 46.95) (layer "Edge.Cuts") (width 0.0381))
 (segment (start 115.09 50) (end 113.08 50) (width 0.25) (layer "F.Cu") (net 3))
 (segment (start 116.08 50.99) (end 115.09 50) (width 0.25) (layer "F.Cu") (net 3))
 (segment (start 108.921 50) (end 113.08 50) (width 0.25) (layer "F.Cu") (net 3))
 (segment (start 116.08 53) (end 116.08 50.99) (width 0.25) (layer "F.Cu") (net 3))
 (via (at 113.08 50) (size 0.6) (drill 0.3) (layers "F.Cu" "B.Cu") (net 3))
 (segment (start 113.08 50) (end 113.08 48) (width 0.25) (layer "B.Cu") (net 3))
 (segment (start 113.08 48) (end 114.08 47) (width 0.25) (layer "B.Cu") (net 3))
 (segment (start 116.08 52.98) (end 118.06 51) (width 0.25) (layer "B.Cu") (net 3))
 (segment (start 108.921 49.35) (end 117.73 49.35) (width 0.25) (layer "F.Cu") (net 2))
 (segment (start 116.08 47) (end 118.08 49) (width 0.25) (layer "B.Cu") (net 2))
 (segment (start 114.08 49) (end 116.08 47) (width 0.25) (layer "B.Cu") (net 2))
 (segment (start 114.08 53) (end 114.08 49) (width 0.25) (layer "B.Cu") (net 2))
 (segment (start 108.921 48.7) (end 116.38 48.7) (width 0.55) (layer "F.Cu") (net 1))
 (segment (start 116.38 48.7) (end 118.08 47) (width 0.55) (layer "F.Cu") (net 1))
 (via (at 110.55 48.6485) (size 0.9) (drill 0.6) (layers "F.Cu" "B.Cu") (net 1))
 (segment (start 112.08 50.1785) (end 112.08 53) (width 0.55) (layer "B.Cu") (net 1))
 (segment (start 110.55 48.6485) (end 112.08 50.1785) (width 0.55) (layer "B.Cu") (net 1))
 (segment (start 110.52 51.3) (end 110.55 51.27) (width 0.25) (layer "F.Cu") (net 4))
 (segment (start 118.08 53) (end 116.72 51.64) (width 0.25) (layer "F.Cu") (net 4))
 (segment (start 108.921 51.3) (end 110.52 51.3) (width 0.25) (layer "F.Cu") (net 4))
 (segment (start 116.72 51.64) (end 116.72 50.17) (width 0.25) (layer "F.Cu") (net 4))
 (via (at 110.25 47.16) (size 0.6) (drill 0.3) (layers "F.Cu" "B.Cu") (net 4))
 (via (at 110.42 52.06) (size 0.6) (drill 0.3) (layers "F.Cu" "B.Cu") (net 4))
 (via (at 110.85 50.79) (size 0.6) (drill 0.3) (layers "F.Cu" "B.Cu") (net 4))
 (via (at 114.76 51.16) (size 0.6) (drill 0.3) (layers "F.Cu" "B.Cu") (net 4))
 (via (at 116.72 50.17) (size 0.6) (drill 0.3) (layers "F.Cu" "B.Cu") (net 4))
 (segment (start 106.221 53.5) (end 108.73 53.5) (width 0.25) (layer "F.Cu") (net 6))
 (segment (start 108.921 46.811) (end 108.61 46.5) (width 0.25) (layer "F.Cu") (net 6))
 (segment (start 108.73 53.5) (end 108.84 53.39) (width 0.25) (layer "F.Cu") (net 6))
 (segment (start 108.921 47.5) (end 108.921 46.811) (width 0.25) (layer "F.Cu") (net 6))
 (segment (start 106.221 53.5) (end 106.221 46.5) (width 0.25) (layer "F.Cu") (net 6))
 (segment (start 108.84 53.39) (end 108.84 52.581) (width 0.25) (layer "F.Cu") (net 6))
 (segment (start 108.61 46.5) (end 106.221 46.5) (width 0.25) (layer "F.Cu") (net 6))
 (segment (start 106.221 53.5) (end 108.75 53.5) (width 0.25) (layer "B.Cu") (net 6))
 (segment (start 108.75 53.5) (end 108.921 53.329) (width 0.25) (layer "B.Cu") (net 6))
 (segment (start 108.921 53.329) (end 108.921 52.5) (width 0.25) (layer "B.Cu") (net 6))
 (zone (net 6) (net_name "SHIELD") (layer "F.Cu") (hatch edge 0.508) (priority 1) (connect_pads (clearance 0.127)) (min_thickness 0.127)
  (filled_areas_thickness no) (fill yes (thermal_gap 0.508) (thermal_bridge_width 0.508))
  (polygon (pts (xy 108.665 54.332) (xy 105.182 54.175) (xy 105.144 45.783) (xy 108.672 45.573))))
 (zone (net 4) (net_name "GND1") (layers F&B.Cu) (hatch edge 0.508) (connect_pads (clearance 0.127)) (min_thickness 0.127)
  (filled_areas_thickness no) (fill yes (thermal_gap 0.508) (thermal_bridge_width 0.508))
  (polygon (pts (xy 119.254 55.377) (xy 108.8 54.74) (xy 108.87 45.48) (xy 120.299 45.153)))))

